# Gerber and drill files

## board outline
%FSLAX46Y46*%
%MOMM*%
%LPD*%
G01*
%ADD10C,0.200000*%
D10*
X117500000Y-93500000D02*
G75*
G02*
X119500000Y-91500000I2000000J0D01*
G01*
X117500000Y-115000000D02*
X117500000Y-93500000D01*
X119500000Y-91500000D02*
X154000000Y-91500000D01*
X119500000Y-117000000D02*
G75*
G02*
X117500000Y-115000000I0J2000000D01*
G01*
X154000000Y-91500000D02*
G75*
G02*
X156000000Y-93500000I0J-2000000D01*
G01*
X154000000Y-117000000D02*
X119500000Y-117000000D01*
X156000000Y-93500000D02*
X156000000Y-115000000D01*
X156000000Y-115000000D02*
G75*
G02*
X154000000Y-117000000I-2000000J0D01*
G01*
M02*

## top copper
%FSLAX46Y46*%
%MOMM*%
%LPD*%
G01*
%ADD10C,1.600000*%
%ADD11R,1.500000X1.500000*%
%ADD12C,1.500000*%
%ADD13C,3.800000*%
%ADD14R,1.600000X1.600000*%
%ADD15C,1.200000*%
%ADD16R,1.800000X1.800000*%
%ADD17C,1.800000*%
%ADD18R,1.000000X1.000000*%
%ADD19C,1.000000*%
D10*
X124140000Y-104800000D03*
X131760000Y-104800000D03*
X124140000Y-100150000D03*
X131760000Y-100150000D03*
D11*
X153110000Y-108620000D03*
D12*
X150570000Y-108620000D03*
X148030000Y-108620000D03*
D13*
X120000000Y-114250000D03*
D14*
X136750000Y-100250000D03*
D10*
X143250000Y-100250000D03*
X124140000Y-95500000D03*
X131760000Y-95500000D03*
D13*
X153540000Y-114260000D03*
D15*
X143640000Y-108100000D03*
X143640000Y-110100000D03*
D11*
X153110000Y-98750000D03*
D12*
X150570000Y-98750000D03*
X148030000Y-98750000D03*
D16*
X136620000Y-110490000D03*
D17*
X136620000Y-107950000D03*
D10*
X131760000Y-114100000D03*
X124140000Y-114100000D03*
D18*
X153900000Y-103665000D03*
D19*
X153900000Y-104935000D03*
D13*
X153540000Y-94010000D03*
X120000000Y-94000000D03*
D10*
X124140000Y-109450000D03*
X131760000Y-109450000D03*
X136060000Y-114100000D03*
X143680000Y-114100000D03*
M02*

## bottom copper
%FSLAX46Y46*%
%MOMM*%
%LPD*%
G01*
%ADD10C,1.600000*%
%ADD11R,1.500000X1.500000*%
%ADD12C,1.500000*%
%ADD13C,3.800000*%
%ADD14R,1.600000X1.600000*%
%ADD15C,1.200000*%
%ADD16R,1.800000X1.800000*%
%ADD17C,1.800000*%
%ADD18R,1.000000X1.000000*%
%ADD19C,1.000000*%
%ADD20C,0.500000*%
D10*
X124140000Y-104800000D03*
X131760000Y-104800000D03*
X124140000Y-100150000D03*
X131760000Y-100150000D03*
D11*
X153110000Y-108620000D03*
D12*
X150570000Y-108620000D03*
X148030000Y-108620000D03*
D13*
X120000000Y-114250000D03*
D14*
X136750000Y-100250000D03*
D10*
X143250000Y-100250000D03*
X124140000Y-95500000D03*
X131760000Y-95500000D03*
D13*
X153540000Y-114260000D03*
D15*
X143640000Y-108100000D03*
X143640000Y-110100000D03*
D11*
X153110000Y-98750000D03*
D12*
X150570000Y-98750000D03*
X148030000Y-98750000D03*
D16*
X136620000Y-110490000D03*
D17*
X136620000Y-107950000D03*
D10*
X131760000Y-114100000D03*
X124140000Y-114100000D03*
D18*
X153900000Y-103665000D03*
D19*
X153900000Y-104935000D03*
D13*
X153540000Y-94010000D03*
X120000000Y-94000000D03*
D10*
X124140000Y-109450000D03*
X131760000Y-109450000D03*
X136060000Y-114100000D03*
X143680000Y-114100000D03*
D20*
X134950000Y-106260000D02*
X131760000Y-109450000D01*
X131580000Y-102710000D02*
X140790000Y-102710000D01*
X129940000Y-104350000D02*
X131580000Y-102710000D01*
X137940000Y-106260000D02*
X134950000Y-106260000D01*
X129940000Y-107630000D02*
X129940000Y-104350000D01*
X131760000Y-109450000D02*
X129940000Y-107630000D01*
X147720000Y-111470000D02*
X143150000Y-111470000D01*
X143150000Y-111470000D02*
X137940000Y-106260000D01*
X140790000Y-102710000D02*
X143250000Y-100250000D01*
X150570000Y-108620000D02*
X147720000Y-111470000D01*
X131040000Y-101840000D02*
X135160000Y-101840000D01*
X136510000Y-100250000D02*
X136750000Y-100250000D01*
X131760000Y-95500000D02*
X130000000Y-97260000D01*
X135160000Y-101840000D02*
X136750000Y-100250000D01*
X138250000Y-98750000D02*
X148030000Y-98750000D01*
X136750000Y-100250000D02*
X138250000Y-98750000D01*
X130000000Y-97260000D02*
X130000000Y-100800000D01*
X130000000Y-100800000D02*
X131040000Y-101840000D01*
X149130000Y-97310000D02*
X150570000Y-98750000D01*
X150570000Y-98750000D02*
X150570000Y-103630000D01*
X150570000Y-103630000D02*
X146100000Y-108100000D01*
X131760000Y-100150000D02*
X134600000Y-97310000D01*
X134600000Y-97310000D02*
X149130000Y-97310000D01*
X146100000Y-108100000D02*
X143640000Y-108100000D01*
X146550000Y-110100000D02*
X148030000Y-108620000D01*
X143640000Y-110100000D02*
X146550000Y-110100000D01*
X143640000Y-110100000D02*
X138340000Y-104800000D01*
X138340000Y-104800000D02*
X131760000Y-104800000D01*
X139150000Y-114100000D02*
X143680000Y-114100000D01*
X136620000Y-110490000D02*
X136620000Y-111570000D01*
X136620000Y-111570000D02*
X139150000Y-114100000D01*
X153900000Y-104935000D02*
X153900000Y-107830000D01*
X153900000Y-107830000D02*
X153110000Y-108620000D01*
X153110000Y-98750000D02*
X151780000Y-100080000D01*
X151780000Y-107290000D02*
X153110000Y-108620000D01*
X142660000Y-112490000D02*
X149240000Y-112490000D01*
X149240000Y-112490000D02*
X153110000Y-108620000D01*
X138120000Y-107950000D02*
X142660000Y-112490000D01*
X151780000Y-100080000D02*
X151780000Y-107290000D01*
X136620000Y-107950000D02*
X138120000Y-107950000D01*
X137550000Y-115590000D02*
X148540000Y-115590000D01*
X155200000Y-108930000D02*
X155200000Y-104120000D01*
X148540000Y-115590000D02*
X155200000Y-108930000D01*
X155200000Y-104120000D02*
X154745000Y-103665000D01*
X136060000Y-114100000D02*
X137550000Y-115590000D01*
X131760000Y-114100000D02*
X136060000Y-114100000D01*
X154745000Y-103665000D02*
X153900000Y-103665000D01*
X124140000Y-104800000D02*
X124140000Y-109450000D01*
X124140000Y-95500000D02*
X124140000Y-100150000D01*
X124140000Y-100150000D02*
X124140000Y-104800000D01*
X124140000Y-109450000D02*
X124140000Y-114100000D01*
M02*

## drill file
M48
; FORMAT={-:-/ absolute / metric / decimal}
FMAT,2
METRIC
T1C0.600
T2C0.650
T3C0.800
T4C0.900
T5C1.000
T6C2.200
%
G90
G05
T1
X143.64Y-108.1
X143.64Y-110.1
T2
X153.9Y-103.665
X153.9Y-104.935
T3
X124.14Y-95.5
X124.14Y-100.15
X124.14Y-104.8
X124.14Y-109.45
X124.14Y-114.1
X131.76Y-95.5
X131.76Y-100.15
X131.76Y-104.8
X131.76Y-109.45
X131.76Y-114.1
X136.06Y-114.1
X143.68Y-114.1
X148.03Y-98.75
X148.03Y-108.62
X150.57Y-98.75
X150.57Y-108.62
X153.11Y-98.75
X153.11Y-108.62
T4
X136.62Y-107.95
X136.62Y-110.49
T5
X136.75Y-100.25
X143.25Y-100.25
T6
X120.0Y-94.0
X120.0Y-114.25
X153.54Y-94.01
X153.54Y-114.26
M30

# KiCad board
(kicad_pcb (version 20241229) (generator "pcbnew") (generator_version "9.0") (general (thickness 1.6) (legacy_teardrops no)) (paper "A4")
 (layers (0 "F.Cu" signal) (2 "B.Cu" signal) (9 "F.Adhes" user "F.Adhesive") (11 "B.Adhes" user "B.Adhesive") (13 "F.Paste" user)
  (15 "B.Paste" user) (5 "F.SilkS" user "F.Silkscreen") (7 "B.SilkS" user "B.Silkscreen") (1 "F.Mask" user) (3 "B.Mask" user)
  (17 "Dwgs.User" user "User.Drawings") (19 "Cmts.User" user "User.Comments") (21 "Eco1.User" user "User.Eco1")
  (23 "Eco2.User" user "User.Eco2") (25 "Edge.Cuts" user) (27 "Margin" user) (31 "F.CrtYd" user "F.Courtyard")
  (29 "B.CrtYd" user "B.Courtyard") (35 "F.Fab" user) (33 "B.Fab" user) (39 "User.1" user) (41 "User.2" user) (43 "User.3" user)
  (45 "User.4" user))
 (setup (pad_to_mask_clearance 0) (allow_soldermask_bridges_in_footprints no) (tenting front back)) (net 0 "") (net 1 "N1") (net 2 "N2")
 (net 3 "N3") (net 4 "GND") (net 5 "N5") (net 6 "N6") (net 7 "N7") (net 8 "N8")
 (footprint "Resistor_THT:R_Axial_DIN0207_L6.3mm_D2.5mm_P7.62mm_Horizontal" (layer "F.Cu") (at 124.14 104.8)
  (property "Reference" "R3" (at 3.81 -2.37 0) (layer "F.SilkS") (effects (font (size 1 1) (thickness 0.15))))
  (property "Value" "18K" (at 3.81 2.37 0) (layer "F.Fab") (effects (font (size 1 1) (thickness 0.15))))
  (pad "1" thru_hole circle (at 0 0) (size 1.6 1.6) (drill 0.8) (layers "*.Cu" "*.Mask") (remove_unused_layers no) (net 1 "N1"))
  (pad "2" thru_hole circle (at 7.62 0) (size 1.6 1.6) (drill 0.8) (layers "*.Cu" "*.Mask") (remove_unused_layers no) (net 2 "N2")))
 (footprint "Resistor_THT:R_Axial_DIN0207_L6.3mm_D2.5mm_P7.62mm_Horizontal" (layer "F.Cu") (at 124.14 100.15)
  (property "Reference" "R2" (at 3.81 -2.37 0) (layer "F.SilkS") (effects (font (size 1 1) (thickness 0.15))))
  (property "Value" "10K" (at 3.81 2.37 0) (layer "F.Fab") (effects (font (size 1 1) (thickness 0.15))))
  (pad "1" thru_hole circle (at 0 0) (size 1.6 1.6) (drill 0.8) (layers "*.Cu" "*.Mask") (remove_unused_layers no) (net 1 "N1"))
  (pad "2" thru_hole circle (at 7.62 0) (size 1.6 1.6) (drill 0.8) (layers "*.Cu" "*.Mask") (remove_unused_layers no) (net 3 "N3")))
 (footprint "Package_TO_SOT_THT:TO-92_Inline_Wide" (layer "F.Cu") (at 153.11 108.62 180)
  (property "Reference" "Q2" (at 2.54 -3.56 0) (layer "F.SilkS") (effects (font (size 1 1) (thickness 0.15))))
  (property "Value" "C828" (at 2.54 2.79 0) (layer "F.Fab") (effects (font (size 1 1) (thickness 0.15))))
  (pad "1" thru_hole rect (at 0 0 180) (size 1.5 1.5) (drill 0.8) (layers "*.Cu" "*.Mask") (remove_unused_layers no) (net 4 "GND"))
  (pad "2" thru_hole circle (at 2.54 0 180) (size 1.5 1.5) (drill 0.8) (layers "*.Cu" "*.Mask") (remove_unused_layers no) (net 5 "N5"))
  (pad "3" thru_hole circle (at 5.08 0 180) (size 1.5 1.5) (drill 0.8) (layers "*.Cu" "*.Mask") (remove_unused_layers no) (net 2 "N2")))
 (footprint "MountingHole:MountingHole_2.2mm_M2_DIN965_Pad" (layer "F.Cu") (at 120 114.25)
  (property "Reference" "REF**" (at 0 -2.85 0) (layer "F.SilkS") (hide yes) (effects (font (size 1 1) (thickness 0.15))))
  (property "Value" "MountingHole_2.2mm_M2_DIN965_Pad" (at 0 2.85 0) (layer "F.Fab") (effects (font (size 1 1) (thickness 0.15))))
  (pad "1" thru_hole circle (at 0 0) (size 3.8 3.8) (drill 2.2) (layers "*.Cu" "*.Mask") (remove_unused_layers no) (zone_connect 2)))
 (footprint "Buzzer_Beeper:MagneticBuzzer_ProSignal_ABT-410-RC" (layer "F.Cu") (at 136.75 100.25)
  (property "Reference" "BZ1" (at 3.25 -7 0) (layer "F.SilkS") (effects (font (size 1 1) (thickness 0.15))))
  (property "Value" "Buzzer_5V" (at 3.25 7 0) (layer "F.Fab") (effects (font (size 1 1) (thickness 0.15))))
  (pad "1" thru_hole rect (at 0 0) (size 1.6 1.6) (drill 1) (layers "*.Cu" "*.Mask") (remove_unused_layers no) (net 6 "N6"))
  (pad "2" thru_hole circle (at 6.5 0) (size 1.6 1.6) (drill 1) (layers "*.Cu" "*.Mask") (remove_unused_layers no) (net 5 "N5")))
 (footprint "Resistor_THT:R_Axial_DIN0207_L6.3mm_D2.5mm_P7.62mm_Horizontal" (layer "F.Cu") (at 124.14 95.5)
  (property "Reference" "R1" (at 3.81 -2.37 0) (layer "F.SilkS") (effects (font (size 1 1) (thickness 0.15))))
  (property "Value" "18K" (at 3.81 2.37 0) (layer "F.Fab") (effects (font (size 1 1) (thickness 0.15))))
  (pad "1" thru_hole circle (at 0 0) (size 1.6 1.6) (drill 0.8) (layers "*.Cu" "*.Mask") (remove_unused_layers no) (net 1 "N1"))
  (pad "2" thru_hole circle (at 7.62 0) (size 1.6 1.6) (drill 0.8) (layers "*.Cu" "*.Mask") (remove_unused_layers no) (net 6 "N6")))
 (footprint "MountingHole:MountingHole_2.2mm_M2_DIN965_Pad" (layer "F.Cu") (at 153.54 114.26)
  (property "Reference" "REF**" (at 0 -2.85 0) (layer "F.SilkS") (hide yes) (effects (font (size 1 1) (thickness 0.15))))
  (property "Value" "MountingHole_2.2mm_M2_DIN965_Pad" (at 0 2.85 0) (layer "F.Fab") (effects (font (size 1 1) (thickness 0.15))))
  (pad "1" thru_hole circle (at 0 0) (size 3.8 3.8) (drill 2.2) (layers "*.Cu" "*.Mask") (remove_unused_layers no) (zone_connect 2)))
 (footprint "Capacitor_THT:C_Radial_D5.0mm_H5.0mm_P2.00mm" (layer "F.Cu") (at 143.64 108.1 -90)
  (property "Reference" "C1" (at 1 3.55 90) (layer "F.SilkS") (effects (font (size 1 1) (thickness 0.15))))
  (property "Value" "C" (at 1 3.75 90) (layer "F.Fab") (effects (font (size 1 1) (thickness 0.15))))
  (pad "1" thru_hole circle (at 0 0 270) (size 1.2 1.2) (drill 0.6) (layers "*.Cu" "*.Mask") (remove_unused_layers no) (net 3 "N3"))
  (pad "2" thru_hole circle (at 2 0 270) (size 1.2 1.2) (drill 0.6) (layers "*.Cu" "*.Mask") (remove_unused_layers no) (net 2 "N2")))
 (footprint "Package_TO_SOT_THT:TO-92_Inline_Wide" (layer "F.Cu") (at 153.11 98.75 180)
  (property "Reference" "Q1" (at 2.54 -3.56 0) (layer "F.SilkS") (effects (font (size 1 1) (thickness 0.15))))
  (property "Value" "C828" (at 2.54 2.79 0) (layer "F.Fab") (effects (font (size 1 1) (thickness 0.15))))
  (pad "1" thru_hole rect (at 0 0 180) (size 1.5 1.5) (drill 0.8) (layers "*.Cu" "*.Mask") (remove_unused_layers no) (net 4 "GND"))
  (pad "2" thru_hole circle (at 2.54 0 180) (size 1.5 1.5) (drill 0.8) (layers "*.Cu" "*.Mask") (remove_unused_layers no) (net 3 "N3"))
  (pad "3" thru_hole circle (at 5.08 0 180) (size 1.5 1.5) (drill 0.8) (layers "*.Cu" "*.Mask") (remove_unused_layers no) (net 6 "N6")))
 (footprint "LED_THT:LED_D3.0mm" (layer "F.Cu") (at 136.62 110.49 90)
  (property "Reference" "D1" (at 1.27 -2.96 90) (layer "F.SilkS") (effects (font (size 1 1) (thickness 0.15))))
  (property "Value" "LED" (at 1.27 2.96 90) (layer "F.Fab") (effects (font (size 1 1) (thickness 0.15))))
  (pad "1" thru_hole rect (at 0 0 90) (size 1.8 1.8) (drill 0.9) (layers "*.Cu" "*.Mask") (remove_unused_layers no) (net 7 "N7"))
  (pad "2" thru_hole circle (at 2.54 0 90) (size 1.8 1.8) (drill 0.9) (layers "*.Cu" "*.Mask") (remove_unused_layers no) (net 4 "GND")))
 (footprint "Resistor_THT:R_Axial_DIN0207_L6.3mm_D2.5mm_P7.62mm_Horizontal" (layer "F.Cu") (at 131.76 114.1 180)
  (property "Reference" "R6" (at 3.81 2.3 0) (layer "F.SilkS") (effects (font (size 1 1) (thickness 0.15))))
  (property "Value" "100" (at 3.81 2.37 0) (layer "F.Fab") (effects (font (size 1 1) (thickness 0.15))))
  (pad "1" thru_hole circle (at 0 0 180) (size 1.6 1.6) (drill 0.8) (layers "*.Cu" "*.Mask") (remove_unused_layers no) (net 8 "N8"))
  (pad "2" thru_hole circle (at 7.62 0 180) (size 1.6 1.6) (drill 0.8) (layers "*.Cu" "*.Mask") (remove_unused_layers no) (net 1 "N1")))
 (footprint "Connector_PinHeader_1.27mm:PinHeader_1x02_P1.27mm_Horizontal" (layer "F.Cu") (at 153.9 103.665)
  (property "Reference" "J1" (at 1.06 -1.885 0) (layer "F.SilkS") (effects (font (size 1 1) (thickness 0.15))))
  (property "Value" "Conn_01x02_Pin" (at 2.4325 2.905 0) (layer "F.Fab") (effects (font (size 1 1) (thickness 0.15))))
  (pad "1" thru_hole rect (at 0 0) (size 1 1) (drill 0.65) (layers "*.Cu" "*.Mask") (remove_unused_layers no) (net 8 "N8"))
  (pad "2" thru_hole circle (at 0 1.27) (size 1 1) (drill 0.65) (layers "*.Cu" "*.Mask") (remove_unused_layers no) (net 4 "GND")))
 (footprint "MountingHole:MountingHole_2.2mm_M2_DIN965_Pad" (layer "F.Cu") (at 153.54 94.01)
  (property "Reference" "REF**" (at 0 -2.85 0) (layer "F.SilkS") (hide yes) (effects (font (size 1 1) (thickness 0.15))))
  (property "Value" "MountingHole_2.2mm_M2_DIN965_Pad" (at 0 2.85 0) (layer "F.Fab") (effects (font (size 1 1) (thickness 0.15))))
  (pad "1" thru_hole circle (at 0 0) (size 3.8 3.8) (drill 2.2) (layers "*.Cu" "*.Mask") (remove_unused_layers no) (zone_connect 2)))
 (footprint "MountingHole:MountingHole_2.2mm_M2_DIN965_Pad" (layer "F.Cu") (at 120 94)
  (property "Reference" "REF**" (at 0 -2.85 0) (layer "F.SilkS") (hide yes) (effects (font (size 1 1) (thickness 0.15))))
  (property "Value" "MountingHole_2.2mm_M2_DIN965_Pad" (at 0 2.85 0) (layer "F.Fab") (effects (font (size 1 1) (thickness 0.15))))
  (pad "1" thru_hole circle (at 0 0) (size 3.8 3.8) (drill 2.2) (layers "*.Cu" "*.Mask") (remove_unused_layers no) (zone_connect 2)))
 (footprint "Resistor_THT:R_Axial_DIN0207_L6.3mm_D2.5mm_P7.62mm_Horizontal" (layer "F.Cu") (at 124.14 109.45)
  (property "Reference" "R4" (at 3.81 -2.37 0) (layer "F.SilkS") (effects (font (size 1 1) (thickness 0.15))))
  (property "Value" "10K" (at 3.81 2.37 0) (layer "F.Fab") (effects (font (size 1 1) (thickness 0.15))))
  (pad "1" thru_hole circle (at 0 0) (size 1.6 1.6) (drill 0.8) (layers "*.Cu" "*.Mask") (remove_unused_layers no) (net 1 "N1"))
  (pad "2" thru_hole circle (at 7.62 0) (size 1.6 1.6) (drill 0.8) (layers "*.Cu" "*.Mask") (remove_unused_layers no) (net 5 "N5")))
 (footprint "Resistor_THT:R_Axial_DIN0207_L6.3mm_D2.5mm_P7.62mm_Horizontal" (layer "F.Cu") (at 136.06 114.1)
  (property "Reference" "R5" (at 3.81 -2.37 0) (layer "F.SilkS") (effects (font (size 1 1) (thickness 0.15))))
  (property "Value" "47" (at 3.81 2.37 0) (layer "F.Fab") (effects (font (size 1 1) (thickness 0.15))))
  (pad "1" thru_hole circle (at 0 0) (size 1.6 1.6) (drill 0.8) (layers "*.Cu" "*.Mask") (remove_unused_layers no) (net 8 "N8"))
  (pad "2" thru_hole circle (at 7.62 0) (size 1.6 1.6) (drill 0.8) (layers "*.Cu" "*.Mask") (remove_unused_layers no) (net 7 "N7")))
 (gr_arc (start 117.5 93.5) (mid 118.085786 92.085786) (end 119.5 91.5) (stroke (width 0.2) (type default)) (layer "Edge.Cuts"))
 (gr_line (start 117.5 115) (end 117.5 93.5) (stroke (width 0.2) (type default)) (layer "Edge.Cuts"))
 (gr_line (start 119.5 91.5) (end 154 91.5) (stroke (width 0.2) (type default)) (layer "Edge.Cuts"))
 (gr_arc (start 119.5 117) (mid 118.085786 116.414214) (end 117.5 115) (stroke (width 0.2) (type default)) (layer "Edge.Cuts"))
 (gr_arc (start 154 91.5) (mid 155.414214 92.085786) (end 156 93.5) (stroke (width 0.2) (type default)) (layer "Edge.Cuts"))
 (gr_line (start 154 117) (end 119.5 117) (stroke (width 0.2) (type default)) (layer "Edge.Cuts"))
 (gr_line (start 156 93.5) (end 156 115) (stroke (width 0.2) (type default)) (layer "Edge.Cuts"))
 (gr_arc (start 156 115) (mid 155.414214 116.414214) (end 154 117) (stroke (width 0.2) (type default)) (layer "Edge.Cuts"))
 (segment (start 134.95 106.26) (end 131.76 109.45) (width 0.5) (layer "B.Cu") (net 5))
 (segment (start 131.58 102.71) (end 140.79 102.71) (width 0.5) (layer "B.Cu") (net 5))
 (segment (start 129.94 104.35) (end 131.58 102.71) (width 0.5) (layer "B.Cu") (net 5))
 (segment (start 137.94 106.26) (end 134.95 106.26) (width 0.5) (layer "B.Cu") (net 5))
 (segment (start 129.94 107.63) (end 129.94 104.35) (width 0.5) (layer "B.Cu") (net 5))
 (segment (start 131.76 109.45) (end 129.94 107.63) (width 0.5) (layer "B.Cu") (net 5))
 (segment (start 147.72 111.47) (end 143.15 111.47) (width 0.5) (layer "B.Cu") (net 5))
 (segment (start 143.15 111.47) (end 137.94 106.26) (width 0.5) (layer "B.Cu") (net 5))
 (segment (start 140.79 102.71) (end 143.25 100.25) (width 0.5) (layer "B.Cu") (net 5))
 (segment (start 150.57 108.62) (end 147.72 111.47) (width 0.5) (layer "B.Cu") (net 5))
 (segment (start 131.04 101.84) (end 135.16 101.84) (width 0.5) (layer "B.Cu") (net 6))
 (segment (start 136.51 100.25) (end 136.75 100.25) (width 0.5) (layer "B.Cu") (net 6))
 (segment (start 131.76 95.5) (end 130 97.26) (width 0.5) (layer "B.Cu") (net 6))
 (segment (start 135.16 101.84) (end 136.75 100.25) (width 0.5) (layer "B.Cu") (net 6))
 (segment (start 138.25 98.75) (end 148.03 98.75) (width 0.5) (layer "B.Cu") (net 6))
 (segment (start 136.75 100.25) (end 138.25 98.75) (width 0.5) (layer "B.Cu") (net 6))
 (segment (start 130 97.26) (end 130 100.8) (width 0.5) (layer "B.Cu") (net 6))
 (segment (start 130 100.8) (end 131.04 101.84) (width 0.5) (layer "B.Cu") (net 6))
 (segment (start 149.13 97.31) (end 150.57 98.75) (width 0.5) (layer "B.Cu") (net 3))
 (segment (start 150.57 98.75) (end 150.57 103.63) (width 0.5) (layer "B.Cu") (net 3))
 (segment (start 150.57 103.63) (end 146.1 108.1) (width 0.5) (layer "B.Cu") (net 3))
 (segment (start 131.76 100.15) (end 134.6 97.31) (width 0.5) (layer "B.Cu") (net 3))
 (segment (start 134.6 97.31) (end 149.13 97.31) (width 0.5) (layer "B.Cu") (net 3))
 (segment (start 146.1 108.1) (end 143.64 108.1) (width 0.5) (layer "B.Cu") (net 3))
 (segment (start 146.55 110.1) (end 148.03 108.62) (width 0.5) (layer "B.Cu") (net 2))
 (segment (start 143.64 110.1) (end 146.55 110.1) (width 0.5) (layer "B.Cu") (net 2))
 (segment (start 143.64 110.1) (end 138.34 104.8) (width 0.5) (layer "B.Cu") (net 2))
 (segment (start 138.34 104.8) (end 131.76 104.8) (width 0.5) (layer "B.Cu") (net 2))
 (segment (start 139.15 114.1) (end 143.68 114.1) (width 0.5) (layer "B.Cu") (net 7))
 (segment (start 136.62 110.49) (end 136.62 111.57) (width 0.5) (layer "B.Cu") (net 7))
 (segment (start 136.62 111.57) (end 139.15 114.1) (width 0.5) (layer "B.Cu") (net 7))
 (segment (start 153.9 104.935) (end 153.9 107.83) (width 0.5) (layer "B.Cu") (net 4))
 (segment (start 153.9 107.83) (end 153.11 108.62) (width 0.5) (layer "B.Cu") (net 4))
 (segment (start 153.11 98.75) (end 151.78 100.08) (width 0.5) (layer "B.Cu") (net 4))
 (segment (start 151.78 107.29) (end 153.11 108.62) (width 0.5) (layer "B.Cu") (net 4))
 (segment (start 142.66 112.49) (end 149.24 112.49) (width 0.5) (layer "B.Cu") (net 4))
 (segment (start 149.24 112.49) (end 153.11 108.62) (width 0.5) (layer "B.Cu") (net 4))
 (segment (start 138.12 107.95) (end 142.66 112.49) (width 0.5) (layer "B.Cu") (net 4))
 (segment (start 151.78 100.08) (end 151.78 107.29) (width 0.5) (layer "B.Cu") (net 4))
 (segment (start 136.62 107.95) (end 138.12 107.95) (width 0.5) (layer "B.Cu") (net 4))
 (segment (start 137.55 115.59) (end 148.54 115.59) (width 0.5) (layer "B.Cu") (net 8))
 (segment (start 155.2 108.93) (end 155.2 104.12) (width 0.5) (layer "B.Cu") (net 8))
 (segment (start 148.54 115.59) (end 155.2 108.93) (width 0.5) (layer "B.Cu") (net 8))
 (segment (start 155.2 104.12) (end 154.745 103.665) (width 0.5) (layer "B.Cu") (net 8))
 (segment (start 136.06 114.1) (end 137.55 115.59) (width 0.5) (layer "B.Cu") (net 8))
 (segment (start 131.76 114.1) (end 136.06 114.1) (width 0.5) (layer "B.Cu") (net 8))
 (segment (start 154.745 103.665) (end 153.9 103.665) (width 0.5) (layer "B.Cu") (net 8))
 (segment (start 124.14 104.8) (end 124.14 109.45) (width 0.5) (layer "B.Cu") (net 1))
 (segment (start 124.14 95.5) (end 124.14 100.15) (width 0.5) (layer "B.Cu") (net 1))
 (segment (start 124.14 100.15) (end 124.14 104.8) (width 0.5) (layer "B.Cu") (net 1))
 (segment (start 124.14 109.45) (end 124.14 114.1) (width 0.5) (layer "B.Cu") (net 1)))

